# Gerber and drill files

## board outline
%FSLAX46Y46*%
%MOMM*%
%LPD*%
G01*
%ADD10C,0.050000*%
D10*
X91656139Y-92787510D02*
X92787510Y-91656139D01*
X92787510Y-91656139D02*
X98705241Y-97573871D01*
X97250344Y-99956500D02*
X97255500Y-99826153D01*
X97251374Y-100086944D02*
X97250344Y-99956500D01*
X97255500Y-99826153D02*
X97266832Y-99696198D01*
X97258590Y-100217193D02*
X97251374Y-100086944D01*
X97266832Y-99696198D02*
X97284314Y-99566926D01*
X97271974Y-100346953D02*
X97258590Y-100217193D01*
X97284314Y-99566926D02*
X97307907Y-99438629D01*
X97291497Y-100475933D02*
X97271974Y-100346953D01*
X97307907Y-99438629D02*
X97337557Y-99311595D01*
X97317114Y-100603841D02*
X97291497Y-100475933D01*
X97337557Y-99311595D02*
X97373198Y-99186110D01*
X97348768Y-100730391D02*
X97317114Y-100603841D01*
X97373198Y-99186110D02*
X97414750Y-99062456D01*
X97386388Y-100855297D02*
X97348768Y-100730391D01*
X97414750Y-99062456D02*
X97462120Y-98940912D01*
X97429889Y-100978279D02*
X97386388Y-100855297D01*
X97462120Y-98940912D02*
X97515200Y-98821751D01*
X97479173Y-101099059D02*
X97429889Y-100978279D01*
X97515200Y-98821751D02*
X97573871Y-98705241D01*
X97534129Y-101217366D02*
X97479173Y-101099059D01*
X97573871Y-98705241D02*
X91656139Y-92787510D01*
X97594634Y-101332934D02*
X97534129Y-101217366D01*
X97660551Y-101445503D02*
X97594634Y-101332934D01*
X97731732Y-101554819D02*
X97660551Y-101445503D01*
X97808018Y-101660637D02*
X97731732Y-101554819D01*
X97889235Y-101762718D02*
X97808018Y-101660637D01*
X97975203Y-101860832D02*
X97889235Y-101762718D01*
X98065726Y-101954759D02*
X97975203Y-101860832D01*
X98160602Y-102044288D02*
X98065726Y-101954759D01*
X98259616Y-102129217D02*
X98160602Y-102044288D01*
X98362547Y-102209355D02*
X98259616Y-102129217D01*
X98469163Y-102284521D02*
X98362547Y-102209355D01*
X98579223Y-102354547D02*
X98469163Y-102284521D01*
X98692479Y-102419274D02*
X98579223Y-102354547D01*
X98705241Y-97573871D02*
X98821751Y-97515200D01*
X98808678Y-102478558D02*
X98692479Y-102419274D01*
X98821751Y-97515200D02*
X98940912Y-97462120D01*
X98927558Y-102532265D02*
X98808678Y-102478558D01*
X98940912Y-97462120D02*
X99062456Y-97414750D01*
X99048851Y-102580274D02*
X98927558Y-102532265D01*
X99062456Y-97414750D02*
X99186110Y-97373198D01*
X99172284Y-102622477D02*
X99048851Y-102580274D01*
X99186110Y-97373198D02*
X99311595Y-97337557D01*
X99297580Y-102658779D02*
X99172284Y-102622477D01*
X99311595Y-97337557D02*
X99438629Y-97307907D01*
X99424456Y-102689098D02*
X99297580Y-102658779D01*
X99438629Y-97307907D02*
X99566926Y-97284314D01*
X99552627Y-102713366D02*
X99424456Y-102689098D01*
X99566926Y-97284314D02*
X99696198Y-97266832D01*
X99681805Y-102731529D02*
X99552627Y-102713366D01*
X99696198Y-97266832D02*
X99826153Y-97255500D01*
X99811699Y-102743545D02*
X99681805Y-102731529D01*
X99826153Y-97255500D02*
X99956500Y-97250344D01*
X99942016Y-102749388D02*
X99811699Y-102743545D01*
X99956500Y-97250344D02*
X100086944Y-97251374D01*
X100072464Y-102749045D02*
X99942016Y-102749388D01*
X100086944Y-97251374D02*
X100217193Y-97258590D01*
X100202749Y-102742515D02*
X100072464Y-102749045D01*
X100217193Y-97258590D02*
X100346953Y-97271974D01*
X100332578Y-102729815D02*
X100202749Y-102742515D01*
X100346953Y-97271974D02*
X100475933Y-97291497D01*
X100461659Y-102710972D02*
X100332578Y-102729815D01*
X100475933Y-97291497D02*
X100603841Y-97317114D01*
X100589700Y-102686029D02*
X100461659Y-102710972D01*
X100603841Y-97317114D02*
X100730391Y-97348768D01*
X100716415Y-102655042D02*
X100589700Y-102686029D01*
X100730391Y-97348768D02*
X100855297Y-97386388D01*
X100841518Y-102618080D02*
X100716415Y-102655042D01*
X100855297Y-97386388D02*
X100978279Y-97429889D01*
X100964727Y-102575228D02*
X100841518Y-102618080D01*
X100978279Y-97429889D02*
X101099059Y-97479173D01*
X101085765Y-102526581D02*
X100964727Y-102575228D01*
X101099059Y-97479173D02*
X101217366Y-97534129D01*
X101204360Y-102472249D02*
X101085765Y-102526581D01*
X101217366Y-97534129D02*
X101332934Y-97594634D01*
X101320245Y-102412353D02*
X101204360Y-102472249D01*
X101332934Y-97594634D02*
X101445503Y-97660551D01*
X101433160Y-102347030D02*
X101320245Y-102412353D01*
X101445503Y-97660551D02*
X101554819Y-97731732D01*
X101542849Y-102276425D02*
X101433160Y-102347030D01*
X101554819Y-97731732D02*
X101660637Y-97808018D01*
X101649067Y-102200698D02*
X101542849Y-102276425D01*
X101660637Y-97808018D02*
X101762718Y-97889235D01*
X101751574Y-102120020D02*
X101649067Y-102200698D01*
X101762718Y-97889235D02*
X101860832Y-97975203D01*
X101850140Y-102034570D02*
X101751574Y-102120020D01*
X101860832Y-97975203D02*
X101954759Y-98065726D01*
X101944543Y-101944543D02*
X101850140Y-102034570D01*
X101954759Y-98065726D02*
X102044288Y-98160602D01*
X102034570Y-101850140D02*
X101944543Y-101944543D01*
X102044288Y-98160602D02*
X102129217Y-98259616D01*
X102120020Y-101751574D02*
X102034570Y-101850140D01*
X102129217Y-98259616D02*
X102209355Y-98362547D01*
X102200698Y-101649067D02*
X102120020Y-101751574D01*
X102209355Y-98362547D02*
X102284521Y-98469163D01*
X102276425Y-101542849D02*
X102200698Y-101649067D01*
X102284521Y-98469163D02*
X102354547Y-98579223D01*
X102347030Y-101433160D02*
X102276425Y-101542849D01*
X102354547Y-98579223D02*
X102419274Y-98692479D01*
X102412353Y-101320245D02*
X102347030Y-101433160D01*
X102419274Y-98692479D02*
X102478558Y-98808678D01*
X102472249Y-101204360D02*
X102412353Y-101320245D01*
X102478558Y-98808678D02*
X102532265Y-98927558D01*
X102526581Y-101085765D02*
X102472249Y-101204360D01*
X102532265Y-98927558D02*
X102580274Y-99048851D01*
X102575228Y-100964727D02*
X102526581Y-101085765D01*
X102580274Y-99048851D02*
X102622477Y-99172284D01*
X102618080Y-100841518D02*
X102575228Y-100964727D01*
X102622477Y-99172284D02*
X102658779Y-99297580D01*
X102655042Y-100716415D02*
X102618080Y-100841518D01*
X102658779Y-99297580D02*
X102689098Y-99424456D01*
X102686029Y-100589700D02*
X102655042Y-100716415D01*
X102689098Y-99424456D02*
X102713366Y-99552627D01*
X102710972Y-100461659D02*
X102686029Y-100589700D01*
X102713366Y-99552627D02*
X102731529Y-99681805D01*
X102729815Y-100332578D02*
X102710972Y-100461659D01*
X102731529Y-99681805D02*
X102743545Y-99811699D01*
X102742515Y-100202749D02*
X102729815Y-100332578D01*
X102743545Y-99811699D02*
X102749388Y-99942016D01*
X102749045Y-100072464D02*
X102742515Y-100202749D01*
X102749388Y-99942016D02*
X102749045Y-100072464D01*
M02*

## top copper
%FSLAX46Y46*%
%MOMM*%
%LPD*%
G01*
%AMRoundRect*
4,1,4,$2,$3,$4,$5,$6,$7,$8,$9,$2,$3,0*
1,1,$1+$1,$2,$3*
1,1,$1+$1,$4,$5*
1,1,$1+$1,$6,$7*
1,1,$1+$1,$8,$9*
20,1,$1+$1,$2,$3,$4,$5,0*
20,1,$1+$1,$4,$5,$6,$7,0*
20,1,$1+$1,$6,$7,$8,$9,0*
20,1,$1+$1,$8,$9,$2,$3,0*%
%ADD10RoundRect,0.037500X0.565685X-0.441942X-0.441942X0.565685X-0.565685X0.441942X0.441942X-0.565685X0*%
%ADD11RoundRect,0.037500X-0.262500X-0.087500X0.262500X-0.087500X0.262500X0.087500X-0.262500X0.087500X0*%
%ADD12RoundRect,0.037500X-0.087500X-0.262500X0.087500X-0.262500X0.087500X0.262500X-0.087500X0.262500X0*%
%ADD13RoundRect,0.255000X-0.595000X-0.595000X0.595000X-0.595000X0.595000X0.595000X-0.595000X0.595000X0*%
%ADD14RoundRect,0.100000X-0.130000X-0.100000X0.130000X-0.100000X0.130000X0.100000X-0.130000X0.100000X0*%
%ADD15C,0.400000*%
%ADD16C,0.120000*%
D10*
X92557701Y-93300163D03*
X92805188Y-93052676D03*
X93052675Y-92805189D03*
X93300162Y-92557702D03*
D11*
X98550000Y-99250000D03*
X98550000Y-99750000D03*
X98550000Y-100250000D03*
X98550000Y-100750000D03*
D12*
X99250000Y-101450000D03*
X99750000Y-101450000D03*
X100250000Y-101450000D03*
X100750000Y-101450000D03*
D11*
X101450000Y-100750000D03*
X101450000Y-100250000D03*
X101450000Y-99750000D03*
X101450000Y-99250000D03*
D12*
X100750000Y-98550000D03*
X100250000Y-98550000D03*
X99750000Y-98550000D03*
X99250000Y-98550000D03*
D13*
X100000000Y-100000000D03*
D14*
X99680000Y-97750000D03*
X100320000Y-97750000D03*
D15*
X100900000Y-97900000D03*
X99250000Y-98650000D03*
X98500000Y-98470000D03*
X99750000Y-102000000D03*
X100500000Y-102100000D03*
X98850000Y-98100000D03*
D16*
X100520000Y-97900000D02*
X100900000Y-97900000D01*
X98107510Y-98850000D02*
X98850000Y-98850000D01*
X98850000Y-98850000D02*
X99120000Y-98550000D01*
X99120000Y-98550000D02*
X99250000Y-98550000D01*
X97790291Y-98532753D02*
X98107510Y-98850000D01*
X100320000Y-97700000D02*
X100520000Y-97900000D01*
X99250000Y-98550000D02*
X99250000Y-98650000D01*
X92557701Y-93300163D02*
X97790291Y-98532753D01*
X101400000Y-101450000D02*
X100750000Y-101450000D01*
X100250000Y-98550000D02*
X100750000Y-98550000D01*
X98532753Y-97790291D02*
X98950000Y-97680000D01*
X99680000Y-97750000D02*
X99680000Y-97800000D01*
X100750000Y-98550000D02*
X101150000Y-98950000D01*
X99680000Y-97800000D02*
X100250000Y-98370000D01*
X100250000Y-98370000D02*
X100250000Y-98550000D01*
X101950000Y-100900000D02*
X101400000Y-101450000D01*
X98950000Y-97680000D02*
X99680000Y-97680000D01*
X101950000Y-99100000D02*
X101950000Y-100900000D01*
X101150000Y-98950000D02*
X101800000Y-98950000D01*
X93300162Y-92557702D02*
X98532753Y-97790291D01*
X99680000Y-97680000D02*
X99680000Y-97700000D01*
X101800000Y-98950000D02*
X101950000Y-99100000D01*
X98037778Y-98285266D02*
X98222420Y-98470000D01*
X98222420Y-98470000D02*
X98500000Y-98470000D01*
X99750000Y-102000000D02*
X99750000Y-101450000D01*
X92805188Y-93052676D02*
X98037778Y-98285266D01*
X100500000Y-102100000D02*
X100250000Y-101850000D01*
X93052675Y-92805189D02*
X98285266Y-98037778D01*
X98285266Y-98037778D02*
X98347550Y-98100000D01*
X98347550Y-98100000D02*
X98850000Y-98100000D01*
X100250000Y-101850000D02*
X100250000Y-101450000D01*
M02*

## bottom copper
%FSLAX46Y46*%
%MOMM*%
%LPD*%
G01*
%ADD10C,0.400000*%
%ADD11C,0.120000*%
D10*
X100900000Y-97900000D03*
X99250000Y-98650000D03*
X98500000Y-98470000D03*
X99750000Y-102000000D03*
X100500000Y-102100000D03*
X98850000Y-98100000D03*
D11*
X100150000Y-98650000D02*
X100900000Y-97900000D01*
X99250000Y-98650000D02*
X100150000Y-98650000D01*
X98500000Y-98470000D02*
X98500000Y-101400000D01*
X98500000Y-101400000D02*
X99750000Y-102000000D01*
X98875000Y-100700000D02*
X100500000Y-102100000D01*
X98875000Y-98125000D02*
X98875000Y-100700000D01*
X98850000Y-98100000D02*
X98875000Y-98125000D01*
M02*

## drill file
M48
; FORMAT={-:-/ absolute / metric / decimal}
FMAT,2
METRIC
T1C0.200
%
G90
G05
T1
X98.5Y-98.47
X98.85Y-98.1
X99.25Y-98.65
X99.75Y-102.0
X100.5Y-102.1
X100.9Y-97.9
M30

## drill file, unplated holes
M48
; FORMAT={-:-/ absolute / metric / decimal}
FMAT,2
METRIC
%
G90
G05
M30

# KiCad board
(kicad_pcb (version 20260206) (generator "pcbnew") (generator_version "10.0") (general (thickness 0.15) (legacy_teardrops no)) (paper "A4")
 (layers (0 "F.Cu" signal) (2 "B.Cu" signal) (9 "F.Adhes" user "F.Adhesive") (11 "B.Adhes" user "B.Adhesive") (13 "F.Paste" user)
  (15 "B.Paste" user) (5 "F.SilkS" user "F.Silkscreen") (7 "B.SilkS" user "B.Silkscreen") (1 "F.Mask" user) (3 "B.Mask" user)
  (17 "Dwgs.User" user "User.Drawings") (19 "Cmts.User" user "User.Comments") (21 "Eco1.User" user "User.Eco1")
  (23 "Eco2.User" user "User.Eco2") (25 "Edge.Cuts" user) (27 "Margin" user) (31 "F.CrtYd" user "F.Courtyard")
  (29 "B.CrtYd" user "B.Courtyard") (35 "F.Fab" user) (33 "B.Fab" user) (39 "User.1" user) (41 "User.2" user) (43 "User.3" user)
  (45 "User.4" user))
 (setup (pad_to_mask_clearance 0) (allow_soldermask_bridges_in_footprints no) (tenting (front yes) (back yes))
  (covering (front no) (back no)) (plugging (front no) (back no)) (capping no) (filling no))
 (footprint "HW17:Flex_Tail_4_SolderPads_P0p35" (layer "F.Cu") (at 92.928932 92.928932 135)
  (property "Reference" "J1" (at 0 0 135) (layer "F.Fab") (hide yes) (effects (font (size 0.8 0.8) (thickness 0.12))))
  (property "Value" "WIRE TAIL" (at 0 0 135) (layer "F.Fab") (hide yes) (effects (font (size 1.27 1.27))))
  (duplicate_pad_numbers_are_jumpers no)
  (pad "1" smd roundrect (at 0 -0.525 135) (size 1.5 0.25) (layers "F.Cu" "F.Mask") (roundrect_rratio 0.15) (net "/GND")
   (solder_mask_margin 0.025) (thermal_bridge_angle 45))
  (pad "2" smd roundrect (at 0 -0.175 135) (size 1.5 0.25) (layers "F.Cu" "F.Mask") (roundrect_rratio 0.15) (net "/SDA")
   (solder_mask_margin 0.025) (thermal_bridge_angle 45))
  (pad "3" smd roundrect (at 0 0.174999 135) (size 1.5 0.25) (layers "F.Cu" "F.Mask") (roundrect_rratio 0.15) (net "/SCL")
   (solder_mask_margin 0.025) (thermal_bridge_angle 45))
  (pad "4" smd roundrect (at 0 0.524999 135) (size 1.5 0.25) (layers "F.Cu" "F.Mask") (roundrect_rratio 0.15) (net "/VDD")
   (solder_mask_margin 0.025) (thermal_bridge_angle 45)))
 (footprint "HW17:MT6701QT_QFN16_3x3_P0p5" (layer "F.Cu") (at 100 100)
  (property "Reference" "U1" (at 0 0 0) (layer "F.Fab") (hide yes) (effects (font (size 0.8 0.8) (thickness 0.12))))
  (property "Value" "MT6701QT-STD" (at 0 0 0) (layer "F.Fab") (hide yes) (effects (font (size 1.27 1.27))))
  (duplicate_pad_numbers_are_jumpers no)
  (pad "" smd roundrect (at -0.4 -0.4) (size 0.65 0.65) (layers "F.Paste") (roundrect_rratio 0.15) (solder_mask_margin 0.025)
   (thermal_bridge_angle 45))
  (pad "" smd roundrect (at -0.4 0.4) (size 0.65 0.65) (layers "F.Paste") (roundrect_rratio 0.15) (solder_mask_margin 0.025)
   (thermal_bridge_angle 45))
  (pad "" smd roundrect (at 0.4 -0.4) (size 0.65 0.65) (layers "F.Paste") (roundrect_rratio 0.15) (solder_mask_margin 0.025)
   (thermal_bridge_angle 45))
  (pad "" smd roundrect (at 0.4 0.4) (size 0.65 0.65) (layers "F.Paste") (roundrect_rratio 0.15) (solder_mask_margin 0.025)
   (thermal_bridge_angle 45))
  (pad "1" smd roundrect (at -1.45 -0.75) (size 0.6 0.25) (layers "F.Cu" "F.Mask" "F.Paste") (roundrect_rratio 0.15)
   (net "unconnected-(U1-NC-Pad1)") (solder_mask_margin 0.025) (thermal_bridge_angle 45))
  (pad "2" smd roundrect (at -1.45 -0.25) (size 0.6 0.25) (layers "F.Cu" "F.Mask" "F.Paste") (roundrect_rratio 0.15)
   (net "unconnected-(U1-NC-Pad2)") (solder_mask_margin 0.025) (thermal_bridge_angle 45))
  (pad "3" smd roundrect (at -1.45 0.25) (size 0.6 0.25) (layers "F.Cu" "F.Mask" "F.Paste") (roundrect_rratio 0.15)
   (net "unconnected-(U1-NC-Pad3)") (solder_mask_margin 0.025) (thermal_bridge_angle 45))
  (pad "4" smd roundrect (at -1.45 0.75) (size 0.6 0.25) (layers "F.Cu" "F.Mask" "F.Paste") (roundrect_rratio 0.15)
   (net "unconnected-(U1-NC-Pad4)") (solder_mask_margin 0.025) (thermal_bridge_angle 45))
  (pad "5" smd roundrect (at -0.75 1.45) (size 0.25 0.6) (layers "F.Cu" "F.Mask" "F.Paste") (roundrect_rratio 0.15)
   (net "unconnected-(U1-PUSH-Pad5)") (solder_mask_margin 0.025) (thermal_bridge_angle 45))
  (pad "6" smd roundrect (at -0.25 1.45) (size 0.25 0.6) (layers "F.Cu" "F.Mask" "F.Paste") (roundrect_rratio 0.15) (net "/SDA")
   (solder_mask_margin 0.025) (thermal_bridge_angle 45))
  (pad "7" smd roundrect (at 0.25 1.45) (size 0.25 0.6) (layers "F.Cu" "F.Mask" "F.Paste") (roundrect_rratio 0.15) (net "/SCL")
   (solder_mask_margin 0.025) (thermal_bridge_angle 45))
  (pad "8" smd roundrect (at 0.75 1.45) (size 0.25 0.6) (layers "F.Cu" "F.Mask" "F.Paste") (roundrect_rratio 0.15) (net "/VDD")
   (solder_mask_margin 0.025) (thermal_bridge_angle 45))
  (pad "9" smd roundrect (at 1.45 0.75) (size 0.6 0.25) (layers "F.Cu" "F.Mask" "F.Paste") (roundrect_rratio 0.15)
   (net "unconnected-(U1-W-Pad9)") (solder_mask_margin 0.025) (thermal_bridge_angle 45))
  (pad "10" smd roundrect (at 1.45 0.25) (size 0.6 0.25) (layers "F.Cu" "F.Mask" "F.Paste") (roundrect_rratio 0.15)
   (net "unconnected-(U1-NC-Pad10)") (solder_mask_margin 0.025) (thermal_bridge_angle 45))
  (pad "11" smd roundrect (at 1.45 -0.25) (size 0.6 0.25) (layers "F.Cu" "F.Mask" "F.Paste") (roundrect_rratio 0.15)
   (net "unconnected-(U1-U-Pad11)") (solder_mask_margin 0.025) (thermal_bridge_angle 45))
  (pad "12" smd roundrect (at 1.45 -0.75) (size 0.6 0.25) (layers "F.Cu" "F.Mask" "F.Paste") (roundrect_rratio 0.15)
   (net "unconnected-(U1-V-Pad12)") (solder_mask_margin 0.025) (thermal_bridge_angle 45))
  (pad "13" smd roundrect (at 0.75 -1.45) (size 0.25 0.6) (layers "F.Cu" "F.Mask" "F.Paste") (roundrect_rratio 0.15) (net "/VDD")
   (solder_mask_margin 0.025) (thermal_bridge_angle 45))
  (pad "14" smd roundrect (at 0.25 -1.45) (size 0.25 0.6) (layers "F.Cu" "F.Mask" "F.Paste") (roundrect_rratio 0.15) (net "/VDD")
   (solder_mask_margin 0.025) (thermal_bridge_angle 45))
  (pad "15" smd roundrect (at -0.25 -1.45) (size 0.25 0.6) (layers "F.Cu" "F.Mask" "F.Paste") (roundrect_rratio 0.15)
   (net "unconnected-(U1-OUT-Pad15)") (solder_mask_margin 0.025) (thermal_bridge_angle 45))
  (pad "16" smd roundrect (at -0.75 -1.45) (size 0.25 0.6) (layers "F.Cu" "F.Mask" "F.Paste") (roundrect_rratio 0.15) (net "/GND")
   (solder_mask_margin 0.025) (thermal_bridge_angle 45))
  (pad "17" smd roundrect (at 0 0) (size 1.7 1.7) (layers "F.Cu" "F.Mask") (roundrect_rratio 0.15)
   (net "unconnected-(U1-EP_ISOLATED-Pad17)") (solder_mask_margin 0.025) (thermal_bridge_angle 45)))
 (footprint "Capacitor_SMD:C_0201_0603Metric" (layer "F.Cu") (at 100 97.75)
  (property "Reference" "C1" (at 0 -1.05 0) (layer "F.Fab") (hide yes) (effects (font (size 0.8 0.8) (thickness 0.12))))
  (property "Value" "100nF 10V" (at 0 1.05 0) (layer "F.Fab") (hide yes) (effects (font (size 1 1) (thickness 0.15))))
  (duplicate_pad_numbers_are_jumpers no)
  (pad "" smd roundrect (at -0.345 0) (size 0.318 0.36) (layers "F.Paste") (roundrect_rratio 0.25))
  (pad "" smd roundrect (at 0.345 0) (size 0.318 0.36) (layers "F.Paste") (roundrect_rratio 0.25))
  (pad "1" smd roundrect (at -0.32 0) (size 0.46 0.4) (layers "F.Cu" "F.Mask") (roundrect_rratio 0.25) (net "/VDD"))
  (pad "2" smd roundrect (at 0.32 0) (size 0.46 0.4) (layers "F.Cu" "F.Mask") (roundrect_rratio 0.25) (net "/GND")))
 (gr_line (start 91.656139 92.78751) (end 92.78751 91.656139) (stroke (width 0.05) (type default)) (layer "Edge.Cuts"))
 (gr_line (start 92.78751 91.656139) (end 98.705241 97.573871) (stroke (width 0.05) (type default)) (layer "Edge.Cuts"))
 (gr_line (start 97.250344 99.9565) (end 97.2555 99.826153) (stroke (width 0.05) (type default)) (layer "Edge.Cuts"))
 (gr_line (start 97.251374 100.086944) (end 97.250344 99.9565) (stroke (width 0.05) (type default)) (layer "Edge.Cuts"))
 (gr_line (start 97.2555 99.826153) (end 97.266832 99.696198) (stroke (width 0.05) (type default)) (layer "Edge.Cuts"))
 (gr_line (start 97.25859 100.217193) (end 97.251374 100.086944) (stroke (width 0.05) (type default)) (layer "Edge.Cuts"))
 (gr_line (start 97.266832 99.696198) (end 97.284314 99.566926) (stroke (width 0.05) (type default)) (layer "Edge.Cuts"))
 (gr_line (start 97.271974 100.346953) (end 97.25859 100.217193) (stroke (width 0.05) (type default)) (layer "Edge.Cuts"))
 (gr_line (start 97.284314 99.566926) (end 97.307907 99.438629) (stroke (width 0.05) (type default)) (layer "Edge.Cuts"))
 (gr_line (start 97.291497 100.475933) (end 97.271974 100.346953) (stroke (width 0.05) (type default)) (layer "Edge.Cuts"))
 (gr_line (start 97.307907 99.438629) (end 97.337557 99.311595) (stroke (width 0.05) (type default)) (layer "Edge.Cuts"))
 (gr_line (start 97.317114 100.603841) (end 97.291497 100.475933) (stroke (width 0.05) (type default)) (layer "Edge.Cuts"))
 (gr_line (start 97.337557 99.311595) (end 97.373198 99.18611) (stroke (width 0.05) (type default)) (layer "Edge.Cuts"))
 (gr_line (start 97.348768 100.730391) (end 97.317114 100.603841) (stroke (width 0.05) (type default)) (layer "Edge.Cuts"))
 (gr_line (start 97.373198 99.18611) (end 97.41475 99.062456) (stroke (width 0.05) (type default)) (layer "Edge.Cuts"))
 (gr_line (start 97.386388 100.855297) (end 97.348768 100.730391) (stroke (width 0.05) (type default)) (layer "Edge.Cuts"))
 (gr_line (start 97.41475 99.062456) (end 97.46212 98.940912) (stroke (width 0.05) (type default)) (layer "Edge.Cuts"))
 (gr_line (start 97.429889 100.978279) (end 97.386388 100.855297) (stroke (width 0.05) (type default)) (layer "Edge.Cuts"))
 (gr_line (start 97.46212 98.940912) (end 97.5152 98.821751) (stroke (width 0.05) (type default)) (layer "Edge.Cuts"))
 (gr_line (start 97.479173 101.099059) (end 97.429889 100.978279) (stroke (width 0.05) (type default)) (layer "Edge.Cuts"))
 (gr_line (start 97.5152 98.821751) (end 97.573871 98.705241) (stroke (width 0.05) (type default)) (layer "Edge.Cuts"))
 (gr_line (start 97.534129 101.217366) (end 97.479173 101.099059) (stroke (width 0.05) (type default)) (layer "Edge.Cuts"))
 (gr_line (start 97.573871 98.705241) (end 91.656139 92.78751) (stroke (width 0.05) (type default)) (layer "Edge.Cuts"))
 (gr_line (start 97.594634 101.332934) (end 97.534129 101.217366) (stroke (width 0.05) (type default)) (layer "Edge.Cuts"))
 (gr_line (start 97.660551 101.445503) (end 97.594634 101.332934) (stroke (width 0.05) (type default)) (layer "Edge.Cuts"))
 (gr_line (start 97.731732 101.554819) (end 97.660551 101.445503) (stroke (width 0.05) (type default)) (layer "Edge.Cuts"))
 (gr_line (start 97.808018 101.660637) (end 97.731732 101.554819) (stroke (width 0.05) (type default)) (layer "Edge.Cuts"))
 (gr_line (start 97.889235 101.762718) (end 97.808018 101.660637) (stroke (width 0.05) (type default)) (layer "Edge.Cuts"))
 (gr_line (start 97.975203 101.860832) (end 97.889235 101.762718) (stroke (width 0.05) (type default)) (layer "Edge.Cuts"))
 (gr_line (start 98.065726 101.954759) (end 97.975203 101.860832) (stroke (width 0.05) (type default)) (layer "Edge.Cuts"))
 (gr_line (start 98.160602 102.044288) (end 98.065726 101.954759) (stroke (width 0.05) (type default)) (layer "Edge.Cuts"))
 (gr_line (start 98.259616 102.129217) (end 98.160602 102.044288) (stroke (width 0.05) (type default)) (layer "Edge.Cuts"))
 (gr_line (start 98.362547 102.209355) (end 98.259616 102.129217) (stroke (width 0.05) (type default)) (layer "Edge.Cuts"))
 (gr_line (start 98.469163 102.284521) (end 98.362547 102.209355) (stroke (width 0.05) (type default)) (layer "Edge.Cuts"))
 (gr_line (start 98.579223 102.354547) (end 98.469163 102.284521) (stroke (width 0.05) (type default)) (layer "Edge.Cuts"))
 (gr_line (start 98.692479 102.419274) (end 98.579223 102.354547) (stroke (width 0.05) (type default)) (layer "Edge.Cuts"))
 (gr_line (start 98.705241 97.573871) (end 98.821751 97.5152) (stroke (width 0.05) (type default)) (layer "Edge.Cuts"))
 (gr_line (start 98.808678 102.478558) (end 98.692479 102.419274) (stroke (width 0.05) (type default)) (layer "Edge.Cuts"))
 (gr_line (start 98.821751 97.5152) (end 98.940912 97.46212) (stroke (width 0.05) (type default)) (layer "Edge.Cuts"))
 (gr_line (start 98.927558 102.532265) (end 98.808678 102.478558) (stroke (width 0.05) (type default)) (layer "Edge.Cuts"))
 (gr_line (start 98.940912 97.46212) (end 99.062456 97.41475) (stroke (width 0.05) (type default)) (layer "Edge.Cuts"))
 (gr_line (start 99.048851 102.580274) (end 98.927558 102.532265) (stroke (width 0.05) (type default)) (layer "Edge.Cuts"))
 (gr_line (start 99.062456 97.41475) (end 99.18611 97.373198) (stroke (width 0.05) (type default)) (layer "Edge.Cuts"))
 (gr_line (start 99.172284 102.622477) (end 99.048851 102.580274) (stroke (width 0.05) (type default)) (layer "Edge.Cuts"))
 (gr_line (start 99.18611 97.373198) (end 99.311595 97.337557) (stroke (width 0.05) (type default)) (layer "Edge.Cuts"))
 (gr_line (start 99.29758 102.658779) (end 99.172284 102.622477) (stroke (width 0.05) (type default)) (layer "Edge.Cuts"))
 (gr_line (start 99.311595 97.337557) (end 99.438629 97.307907) (stroke (width 0.05) (type default)) (layer "Edge.Cuts"))
 (gr_line (start 99.424456 102.689098) (end 99.29758 102.658779) (stroke (width 0.05) (type default)) (layer "Edge.Cuts"))
 (gr_line (start 99.438629 97.307907) (end 99.566926 97.284314) (stroke (width 0.05) (type default)) (layer "Edge.Cuts"))
 (gr_line (start 99.552627 102.713366) (end 99.424456 102.689098) (stroke (width 0.05) (type default)) (layer "Edge.Cuts"))
 (gr_line (start 99.566926 97.284314) (end 99.696198 97.266832) (stroke (width 0.05) (type default)) (layer "Edge.Cuts"))
 (gr_line (start 99.681805 102.731529) (end 99.552627 102.713366) (stroke (width 0.05) (type default)) (layer "Edge.Cuts"))
 (gr_line (start 99.696198 97.266832) (end 99.826153 97.2555) (stroke (width 0.05) (type default)) (layer "Edge.Cuts"))
 (gr_line (start 99.811699 102.743545) (end 99.681805 102.731529) (stroke (width 0.05) (type default)) (layer "Edge.Cuts"))
 (gr_line (start 99.826153 97.2555) (end 99.9565 97.250344) (stroke (width 0.05) (type default)) (layer "Edge.Cuts"))
 (gr_line (start 99.942016 102.749388) (end 99.811699 102.743545) (stroke (width 0.05) (type default)) (layer "Edge.Cuts"))
 (gr_line (start 99.9565 97.250344) (end 100.086944 97.251374) (stroke (width 0.05) (type default)) (layer "Edge.Cuts"))
 (gr_line (start 100.072464 102.749045) (end 99.942016 102.749388) (stroke (width 0.05) (type default)) (layer "Edge.Cuts"))
 (gr_line (start 100.086944 97.251374) (end 100.217193 97.25859) (stroke (width 0.05) (type default)) (layer "Edge.Cuts"))
 (gr_line (start 100.202749 102.742515) (end 100.072464 102.749045) (stroke (width 0.05) (type default)) (layer "Edge.Cuts"))
 (gr_line (start 100.217193 97.25859) (end 100.346953 97.271974) (stroke (width 0.05) (type default)) (layer "Edge.Cuts"))
 (gr_line (start 100.332578 102.729815) (end 100.202749 102.742515) (stroke (width 0.05) (type default)) (layer "Edge.Cuts"))
 (gr_line (start 100.346953 97.271974) (end 100.475933 97.291497) (stroke (width 0.05) (type default)) (layer "Edge.Cuts"))
 (gr_line (start 100.461659 102.710972) (end 100.332578 102.729815) (stroke (width 0.05) (type default)) (layer "Edge.Cuts"))
 (gr_line (start 100.475933 97.291497) (end 100.603841 97.317114) (stroke (width 0.05) (type default)) (layer "Edge.Cuts"))
 (gr_line (start 100.5897 102.686029) (end 100.461659 102.710972) (stroke (width 0.05) (type default)) (layer "Edge.Cuts"))
 (gr_line (start 100.603841 97.317114) (end 100.730391 97.348768) (stroke (width 0.05) (type default)) (layer "Edge.Cuts"))
 (gr_line (start 100.716415 102.655042) (end 100.5897 102.686029) (stroke (width 0.05) (type default)) (layer "Edge.Cuts"))
 (gr_line (start 100.730391 97.348768) (end 100.855297 97.386388) (stroke (width 0.05) (type default)) (layer "Edge.Cuts"))
 (gr_line (start 100.841518 102.61808) (end 100.716415 102.655042) (stroke (width 0.05) (type default)) (layer "Edge.Cuts"))
 (gr_line (start 100.855297 97.386388) (end 100.978279 97.429889) (stroke (width 0.05) (type default)) (layer "Edge.Cuts"))
 (gr_line (start 100.964727 102.575228) (end 100.841518 102.61808) (stroke (width 0.05) (type default)) (layer "Edge.Cuts"))
 (gr_line (start 100.978279 97.429889) (end 101.099059 97.479173) (stroke (width 0.05) (type default)) (layer "Edge.Cuts"))
 (gr_line (start 101.085765 102.526581) (end 100.964727 102.575228) (stroke (width 0.05) (type default)) (layer "Edge.Cuts"))
 (gr_line (start 101.099059 97.479173) (end 101.217366 97.534129) (stroke (width 0.05) (type default)) (layer "Edge.Cuts"))
 (gr_line (start 101.20436 102.472249) (end 101.085765 102.526581) (stroke (width 0.05) (type default)) (layer "Edge.Cuts"))
 (gr_line (start 101.217366 97.534129) (end 101.332934 97.594634) (stroke (width 0.05) (type default)) (layer "Edge.Cuts"))
 (gr_line (start 101.320245 102.412353) (end 101.20436 102.472249) (stroke (width 0.05) (type default)) (layer "Edge.Cuts"))
 (gr_line (start 101.332934 97.594634) (end 101.445503 97.660551) (stroke (width 0.05) (type default)) (layer "Edge.Cuts"))
 (gr_line (start 101.43316 102.34703) (end 101.320245 102.412353) (stroke (width 0.05) (type default)) (layer "Edge.Cuts"))
 (gr_line (start 101.445503 97.660551) (end 101.554819 97.731732) (stroke (width 0.05) (type default)) (layer "Edge.Cuts"))
 (gr_line (start 101.542849 102.276425) (end 101.43316 102.34703) (stroke (width 0.05) (type default)) (layer "Edge.Cuts"))
 (gr_line (start 101.554819 97.731732) (end 101.660637 97.808018) (stroke (width 0.05) (type default)) (layer "Edge.Cuts"))
 (gr_line (start 101.649067 102.200698) (end 101.542849 102.276425) (stroke (width 0.05) (type default)) (layer "Edge.Cuts"))
 (gr_line (start 101.660637 97.808018) (end 101.762718 97.889235) (stroke (width 0.05) (type default)) (layer "Edge.Cuts"))
 (gr_line (start 101.751574 102.12002) (end 101.649067 102.200698) (stroke (width 0.05) (type default)) (layer "Edge.Cuts"))
 (gr_line (start 101.762718 97.889235) (end 101.860832 97.975203) (stroke (width 0.05) (type default)) (layer "Edge.Cuts"))
 (gr_line (start 101.85014 102.03457) (end 101.751574 102.12002) (stroke (width 0.05) (type default)) (layer "Edge.Cuts"))
 (gr_line (start 101.860832 97.975203) (end 101.954759 98.065726) (stroke (width 0.05) (type default)) (layer "Edge.Cuts"))
 (gr_line (start 101.944543 101.944543) (end 101.85014 102.03457) (stroke (width 0.05) (type default)) (layer "Edge.Cuts"))
 (gr_line (start 101.954759 98.065726) (end 102.044288 98.160602) (stroke (width 0.05) (type default)) (layer "Edge.Cuts"))
 (gr_line (start 102.03457 101.85014) (end 101.944543 101.944543) (stroke (width 0.05) (type default)) (layer "Edge.Cuts"))
 (gr_line (start 102.044288 98.160602) (end 102.129217 98.259616) (stroke (width 0.05) (type default)) (layer "Edge.Cuts"))
 (gr_line (start 102.12002 101.751574) (end 102.03457 101.85014) (stroke (width 0.05) (type default)) (layer "Edge.Cuts"))
 (gr_line (start 102.129217 98.259616) (end 102.209355 98.362547) (stroke (width 0.05) (type default)) (layer "Edge.Cuts"))
 (gr_line (start 102.200698 101.649067) (end 102.12002 101.751574) (stroke (width 0.05) (type default)) (layer "Edge.Cuts"))
 (gr_line (start 102.209355 98.362547) (end 102.284521 98.469163) (stroke (width 0.05) (type default)) (layer "Edge.Cuts"))
 (gr_line (start 102.276425 101.542849) (end 102.200698 101.649067) (stroke (width 0.05) (type default)) (layer "Edge.Cuts"))
 (gr_line (start 102.284521 98.469163) (end 102.354547 98.579223) (stroke (width 0.05) (type default)) (layer "Edge.Cuts"))
 (gr_line (start 102.34703 101.43316) (end 102.276425 101.542849) (stroke (width 0.05) (type default)) (layer "Edge.Cuts"))
 (gr_line (start 102.354547 98.579223) (end 102.419274 98.692479) (stroke (width 0.05) (type default)) (layer "Edge.Cuts"))
 (gr_line (start 102.412353 101.320245) (end 102.34703 101.43316) (stroke (width 0.05) (type default)) (layer "Edge.Cuts"))
 (gr_line (start 102.419274 98.692479) (end 102.478558 98.808678) (stroke (width 0.05) (type default)) (layer "Edge.Cuts"))
 (gr_line (start 102.472249 101.20436) (end 102.412353 101.320245) (stroke (width 0.05) (type default)) (layer "Edge.Cuts"))
 (gr_line (start 102.478558 98.808678) (end 102.532265 98.927558) (stroke (width 0.05) (type default)) (layer "Edge.Cuts"))
 (gr_line (start 102.526581 101.085765) (end 102.472249 101.20436) (stroke (width 0.05) (type default)) (layer "Edge.Cuts"))
 (gr_line (start 102.532265 98.927558) (end 102.580274 99.048851) (stroke (width 0.05) (type default)) (layer "Edge.Cuts"))
 (gr_line (start 102.575228 100.964727) (end 102.526581 101.085765) (stroke (width 0.05) (type default)) (layer "Edge.Cuts"))
 (gr_line (start 102.580274 99.048851) (end 102.622477 99.172284) (stroke (width 0.05) (type default)) (layer "Edge.Cuts"))
 (gr_line (start 102.61808 100.841518) (end 102.575228 100.964727) (stroke (width 0.05) (type default)) (layer "Edge.Cuts"))
 (gr_line (start 102.622477 99.172284) (end 102.658779 99.29758) (stroke (width 0.05) (type default)) (layer "Edge.Cuts"))
 (gr_line (start 102.655042 100.716415) (end 102.61808 100.841518) (stroke (width 0.05) (type default)) (layer "Edge.Cuts"))
 (gr_line (start 102.658779 99.29758) (end 102.689098 99.424456) (stroke (width 0.05) (type default)) (layer "Edge.Cuts"))
 (gr_line (start 102.686029 100.5897) (end 102.655042 100.716415) (stroke (width 0.05) (type default)) (layer "Edge.Cuts"))
 (gr_line (start 102.689098 99.424456) (end 102.713366 99.552627) (stroke (width 0.05) (type default)) (layer "Edge.Cuts"))
 (gr_line (start 102.710972 100.461659) (end 102.686029 100.5897) (stroke (width 0.05) (type default)) (layer "Edge.Cuts"))
 (gr_line (start 102.713366 99.552627) (end 102.731529 99.681805) (stroke (width 0.05) (type default)) (layer "Edge.Cuts"))
 (gr_line (start 102.729815 100.332578) (end 102.710972 100.461659) (stroke (width 0.05) (type default)) (layer "Edge.Cuts"))
 (gr_line (start 102.731529 99.681805) (end 102.743545 99.811699) (stroke (width 0.05) (type default)) (layer "Edge.Cuts"))
 (gr_line (start 102.742515 100.202749) (end 102.729815 100.332578) (stroke (width 0.05) (type default)) (layer "Edge.Cuts"))
 (gr_line (start 102.743545 99.811699) (end 102.749388 99.942016) (stroke (width 0.05) (type default)) (layer "Edge.Cuts"))
 (gr_line (start 102.749045 100.072464) (end 102.742515 100.202749) (stroke (width 0.05) (type default)) (layer "Edge.Cuts"))
 (gr_line (start 102.749388 99.942016) (end 102.749045 100.072464) (stroke (width 0.05) (type default)) (layer "Edge.Cuts"))
 (segment (start 100.52 97.9) (end 100.9 97.9) (width 0.12) (locked yes) (layer "F.Cu") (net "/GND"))
 (segment (start 98.10751 98.85) (end 98.85 98.85) (width 0.12) (locked yes) (layer "F.Cu") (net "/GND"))
 (segment (start 98.85 98.85) (end 99.12 98.55) (width 0.12) (locked yes) (layer "F.Cu") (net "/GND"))
 (segment (start 99.12 98.55) (end 99.25 98.55) (width 0.12) (locked yes) (layer "F.Cu") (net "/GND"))
 (segment (start 97.790291 98.532753) (end 98.10751 98.85) (width 0.12) (locked yes) (layer "F.Cu") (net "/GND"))
 (segment (start 100.32 97.7) (end 100.52 97.9) (width 0.12) (locked yes) (layer "F.Cu") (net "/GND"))
 (segment (start 99.25 98.55) (end 99.25 98.65) (width 0.12) (locked yes) (layer "F.Cu") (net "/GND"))
 (segment (start 92.557701 93.300163) (end 97.790291 98.532753) (width 0.12) (locked yes) (layer "F.Cu") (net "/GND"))
 (via (at 100.9 97.9) (size 0.4) (drill 0.2) (layers "F.Cu" "B.Cu") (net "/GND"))
 (via (at 99.25 98.65) (size 0.4) (drill 0.2) (layers "F.Cu" "B.Cu") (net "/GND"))
 (segment (start 100.15 98.65) (end 100.9 97.9) (width 0.12) (locked yes) (layer "B.Cu") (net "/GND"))
 (segment (start 99.25 98.65) (end 100.15 98.65) (width 0.12) (locked yes) (layer "B.Cu") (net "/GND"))
 (segment (start 101.4 101.45) (end 100.75 101.45) (width 0.12) (locked yes) (layer "F.Cu") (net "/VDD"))
 (segment (start 100.25 98.55) (end 100.75 98.55) (width 0.12) (locked yes) (layer "F.Cu") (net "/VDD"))
 (segment (start 98.532753 97.790291) (end 98.95 97.68) (width 0.12) (locked yes) (layer "F.Cu") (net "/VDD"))
 (segment (start 99.68 97.75) (end 99.68 97.8) (width 0.12) (locked yes) (layer "F.Cu") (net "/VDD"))
 (segment (start 100.75 98.55) (end 101.15 98.95) (width 0.12) (locked yes) (layer "F.Cu") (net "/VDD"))
 (segment (start 99.68 97.8) (end 100.25 98.37) (width 0.12) (locked yes) (layer "F.Cu") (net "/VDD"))
 (segment (start 100.25 98.37) (end 100.25 98.55) (width 0.12) (locked yes) (layer "F.Cu") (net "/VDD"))
 (segment (start 101.95 100.9) (end 101.4 101.45) (width 0.12) (locked yes) (layer "F.Cu") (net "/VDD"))
 (segment (start 98.95 97.68) (end 99.68 97.68) (width 0.12) (locked yes) (layer "F.Cu") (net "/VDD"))
 (segment (start 101.95 99.1) (end 101.95 100.9) (width 0.12) (locked yes) (layer "F.Cu") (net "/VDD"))
 (segment (start 101.15 98.95) (end 101.8 98.95) (width 0.12) (locked yes) (layer "F.Cu") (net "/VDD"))
 (segment (start 93.300162 92.557702) (end 98.532753 97.790291) (width 0.12) (locked yes) (layer "F.Cu") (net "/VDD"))
 (segment (start 99.68 97.68) (end 99.68 97.7) (width 0.12) (locked yes) (layer "F.Cu") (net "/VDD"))
 (segment (start 101.8 98.95) (end 101.95 99.1) (width 0.12) (locked yes) (layer "F.Cu") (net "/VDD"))
 (segment (start 98.037778 98.285266) (end 98.22242 98.47) (width 0.12) (locked yes) (layer "F.Cu") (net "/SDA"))
 (segment (start 98.22242 98.47) (end 98.5 98.47) (width 0.12) (locked yes) (layer "F.Cu") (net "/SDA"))
 (segment (start 99.75 102) (end 99.75 101.45) (width 0.12) (locked yes) (layer "F.Cu") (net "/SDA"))
 (segment (start 92.805188 93.052676) (end 98.037778 98.285266) (width 0.12) (locked yes) (layer "F.Cu") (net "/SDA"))
 (via (at 98.5 98.47) (size 0.4) (drill 0.2) (layers "F.Cu" "B.Cu") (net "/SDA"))
 (via (at 99.75 102) (size 0.4) (drill 0.2) (layers "F.Cu" "B.Cu") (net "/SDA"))
 (segment (start 98.5 98.47) (end 98.5 101.4) (width 0.12) (locked yes) (layer "B.Cu") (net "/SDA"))
 (segment (start 98.5 101.4) (end 99.75 102) (width 0.12) (locked yes) (layer "B.Cu") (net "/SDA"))
 (segment (start 100.5 102.1) (end 100.25 101.85) (width 0.12) (locked yes) (layer "F.Cu") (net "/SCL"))
 (segment (start 93.052675 92.805189) (end 98.285266 98.037778) (width 0.12) (locked yes) (layer "F.Cu") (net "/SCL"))
 (segment (start 98.285266 98.037778) (end 98.34755 98.1) (width 0.12) (locked yes) (layer "F.Cu") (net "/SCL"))
 (segment (start 98.34755 98.1) (end 98.85 98.1) (width 0.12) (locked yes) (layer "F.Cu") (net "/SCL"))
 (segment (start 100.25 101.85) (end 100.25 101.45) (width 0.12) (locked yes) (layer "F.Cu") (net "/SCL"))
 (via (at 100.5 102.1) (size 0.4) (drill 0.2) (layers "F.Cu" "B.Cu") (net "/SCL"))
 (via (at 98.85 98.1) (size 0.4) (drill 0.2) (layers "F.Cu" "B.Cu") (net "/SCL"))
 (segment (start 98.875 100.7) (end 100.5 102.1) (width 0.12) (locked yes) (layer "B.Cu") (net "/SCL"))
 (segment (start 98.875 98.125) (end 98.875 100.7) (width 0.12) (locked yes) (layer "B.Cu") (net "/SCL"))
 (segment (start 98.85 98.1) (end 98.875 98.125) (width 0.12) (locked yes) (layer "B.Cu") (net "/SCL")))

